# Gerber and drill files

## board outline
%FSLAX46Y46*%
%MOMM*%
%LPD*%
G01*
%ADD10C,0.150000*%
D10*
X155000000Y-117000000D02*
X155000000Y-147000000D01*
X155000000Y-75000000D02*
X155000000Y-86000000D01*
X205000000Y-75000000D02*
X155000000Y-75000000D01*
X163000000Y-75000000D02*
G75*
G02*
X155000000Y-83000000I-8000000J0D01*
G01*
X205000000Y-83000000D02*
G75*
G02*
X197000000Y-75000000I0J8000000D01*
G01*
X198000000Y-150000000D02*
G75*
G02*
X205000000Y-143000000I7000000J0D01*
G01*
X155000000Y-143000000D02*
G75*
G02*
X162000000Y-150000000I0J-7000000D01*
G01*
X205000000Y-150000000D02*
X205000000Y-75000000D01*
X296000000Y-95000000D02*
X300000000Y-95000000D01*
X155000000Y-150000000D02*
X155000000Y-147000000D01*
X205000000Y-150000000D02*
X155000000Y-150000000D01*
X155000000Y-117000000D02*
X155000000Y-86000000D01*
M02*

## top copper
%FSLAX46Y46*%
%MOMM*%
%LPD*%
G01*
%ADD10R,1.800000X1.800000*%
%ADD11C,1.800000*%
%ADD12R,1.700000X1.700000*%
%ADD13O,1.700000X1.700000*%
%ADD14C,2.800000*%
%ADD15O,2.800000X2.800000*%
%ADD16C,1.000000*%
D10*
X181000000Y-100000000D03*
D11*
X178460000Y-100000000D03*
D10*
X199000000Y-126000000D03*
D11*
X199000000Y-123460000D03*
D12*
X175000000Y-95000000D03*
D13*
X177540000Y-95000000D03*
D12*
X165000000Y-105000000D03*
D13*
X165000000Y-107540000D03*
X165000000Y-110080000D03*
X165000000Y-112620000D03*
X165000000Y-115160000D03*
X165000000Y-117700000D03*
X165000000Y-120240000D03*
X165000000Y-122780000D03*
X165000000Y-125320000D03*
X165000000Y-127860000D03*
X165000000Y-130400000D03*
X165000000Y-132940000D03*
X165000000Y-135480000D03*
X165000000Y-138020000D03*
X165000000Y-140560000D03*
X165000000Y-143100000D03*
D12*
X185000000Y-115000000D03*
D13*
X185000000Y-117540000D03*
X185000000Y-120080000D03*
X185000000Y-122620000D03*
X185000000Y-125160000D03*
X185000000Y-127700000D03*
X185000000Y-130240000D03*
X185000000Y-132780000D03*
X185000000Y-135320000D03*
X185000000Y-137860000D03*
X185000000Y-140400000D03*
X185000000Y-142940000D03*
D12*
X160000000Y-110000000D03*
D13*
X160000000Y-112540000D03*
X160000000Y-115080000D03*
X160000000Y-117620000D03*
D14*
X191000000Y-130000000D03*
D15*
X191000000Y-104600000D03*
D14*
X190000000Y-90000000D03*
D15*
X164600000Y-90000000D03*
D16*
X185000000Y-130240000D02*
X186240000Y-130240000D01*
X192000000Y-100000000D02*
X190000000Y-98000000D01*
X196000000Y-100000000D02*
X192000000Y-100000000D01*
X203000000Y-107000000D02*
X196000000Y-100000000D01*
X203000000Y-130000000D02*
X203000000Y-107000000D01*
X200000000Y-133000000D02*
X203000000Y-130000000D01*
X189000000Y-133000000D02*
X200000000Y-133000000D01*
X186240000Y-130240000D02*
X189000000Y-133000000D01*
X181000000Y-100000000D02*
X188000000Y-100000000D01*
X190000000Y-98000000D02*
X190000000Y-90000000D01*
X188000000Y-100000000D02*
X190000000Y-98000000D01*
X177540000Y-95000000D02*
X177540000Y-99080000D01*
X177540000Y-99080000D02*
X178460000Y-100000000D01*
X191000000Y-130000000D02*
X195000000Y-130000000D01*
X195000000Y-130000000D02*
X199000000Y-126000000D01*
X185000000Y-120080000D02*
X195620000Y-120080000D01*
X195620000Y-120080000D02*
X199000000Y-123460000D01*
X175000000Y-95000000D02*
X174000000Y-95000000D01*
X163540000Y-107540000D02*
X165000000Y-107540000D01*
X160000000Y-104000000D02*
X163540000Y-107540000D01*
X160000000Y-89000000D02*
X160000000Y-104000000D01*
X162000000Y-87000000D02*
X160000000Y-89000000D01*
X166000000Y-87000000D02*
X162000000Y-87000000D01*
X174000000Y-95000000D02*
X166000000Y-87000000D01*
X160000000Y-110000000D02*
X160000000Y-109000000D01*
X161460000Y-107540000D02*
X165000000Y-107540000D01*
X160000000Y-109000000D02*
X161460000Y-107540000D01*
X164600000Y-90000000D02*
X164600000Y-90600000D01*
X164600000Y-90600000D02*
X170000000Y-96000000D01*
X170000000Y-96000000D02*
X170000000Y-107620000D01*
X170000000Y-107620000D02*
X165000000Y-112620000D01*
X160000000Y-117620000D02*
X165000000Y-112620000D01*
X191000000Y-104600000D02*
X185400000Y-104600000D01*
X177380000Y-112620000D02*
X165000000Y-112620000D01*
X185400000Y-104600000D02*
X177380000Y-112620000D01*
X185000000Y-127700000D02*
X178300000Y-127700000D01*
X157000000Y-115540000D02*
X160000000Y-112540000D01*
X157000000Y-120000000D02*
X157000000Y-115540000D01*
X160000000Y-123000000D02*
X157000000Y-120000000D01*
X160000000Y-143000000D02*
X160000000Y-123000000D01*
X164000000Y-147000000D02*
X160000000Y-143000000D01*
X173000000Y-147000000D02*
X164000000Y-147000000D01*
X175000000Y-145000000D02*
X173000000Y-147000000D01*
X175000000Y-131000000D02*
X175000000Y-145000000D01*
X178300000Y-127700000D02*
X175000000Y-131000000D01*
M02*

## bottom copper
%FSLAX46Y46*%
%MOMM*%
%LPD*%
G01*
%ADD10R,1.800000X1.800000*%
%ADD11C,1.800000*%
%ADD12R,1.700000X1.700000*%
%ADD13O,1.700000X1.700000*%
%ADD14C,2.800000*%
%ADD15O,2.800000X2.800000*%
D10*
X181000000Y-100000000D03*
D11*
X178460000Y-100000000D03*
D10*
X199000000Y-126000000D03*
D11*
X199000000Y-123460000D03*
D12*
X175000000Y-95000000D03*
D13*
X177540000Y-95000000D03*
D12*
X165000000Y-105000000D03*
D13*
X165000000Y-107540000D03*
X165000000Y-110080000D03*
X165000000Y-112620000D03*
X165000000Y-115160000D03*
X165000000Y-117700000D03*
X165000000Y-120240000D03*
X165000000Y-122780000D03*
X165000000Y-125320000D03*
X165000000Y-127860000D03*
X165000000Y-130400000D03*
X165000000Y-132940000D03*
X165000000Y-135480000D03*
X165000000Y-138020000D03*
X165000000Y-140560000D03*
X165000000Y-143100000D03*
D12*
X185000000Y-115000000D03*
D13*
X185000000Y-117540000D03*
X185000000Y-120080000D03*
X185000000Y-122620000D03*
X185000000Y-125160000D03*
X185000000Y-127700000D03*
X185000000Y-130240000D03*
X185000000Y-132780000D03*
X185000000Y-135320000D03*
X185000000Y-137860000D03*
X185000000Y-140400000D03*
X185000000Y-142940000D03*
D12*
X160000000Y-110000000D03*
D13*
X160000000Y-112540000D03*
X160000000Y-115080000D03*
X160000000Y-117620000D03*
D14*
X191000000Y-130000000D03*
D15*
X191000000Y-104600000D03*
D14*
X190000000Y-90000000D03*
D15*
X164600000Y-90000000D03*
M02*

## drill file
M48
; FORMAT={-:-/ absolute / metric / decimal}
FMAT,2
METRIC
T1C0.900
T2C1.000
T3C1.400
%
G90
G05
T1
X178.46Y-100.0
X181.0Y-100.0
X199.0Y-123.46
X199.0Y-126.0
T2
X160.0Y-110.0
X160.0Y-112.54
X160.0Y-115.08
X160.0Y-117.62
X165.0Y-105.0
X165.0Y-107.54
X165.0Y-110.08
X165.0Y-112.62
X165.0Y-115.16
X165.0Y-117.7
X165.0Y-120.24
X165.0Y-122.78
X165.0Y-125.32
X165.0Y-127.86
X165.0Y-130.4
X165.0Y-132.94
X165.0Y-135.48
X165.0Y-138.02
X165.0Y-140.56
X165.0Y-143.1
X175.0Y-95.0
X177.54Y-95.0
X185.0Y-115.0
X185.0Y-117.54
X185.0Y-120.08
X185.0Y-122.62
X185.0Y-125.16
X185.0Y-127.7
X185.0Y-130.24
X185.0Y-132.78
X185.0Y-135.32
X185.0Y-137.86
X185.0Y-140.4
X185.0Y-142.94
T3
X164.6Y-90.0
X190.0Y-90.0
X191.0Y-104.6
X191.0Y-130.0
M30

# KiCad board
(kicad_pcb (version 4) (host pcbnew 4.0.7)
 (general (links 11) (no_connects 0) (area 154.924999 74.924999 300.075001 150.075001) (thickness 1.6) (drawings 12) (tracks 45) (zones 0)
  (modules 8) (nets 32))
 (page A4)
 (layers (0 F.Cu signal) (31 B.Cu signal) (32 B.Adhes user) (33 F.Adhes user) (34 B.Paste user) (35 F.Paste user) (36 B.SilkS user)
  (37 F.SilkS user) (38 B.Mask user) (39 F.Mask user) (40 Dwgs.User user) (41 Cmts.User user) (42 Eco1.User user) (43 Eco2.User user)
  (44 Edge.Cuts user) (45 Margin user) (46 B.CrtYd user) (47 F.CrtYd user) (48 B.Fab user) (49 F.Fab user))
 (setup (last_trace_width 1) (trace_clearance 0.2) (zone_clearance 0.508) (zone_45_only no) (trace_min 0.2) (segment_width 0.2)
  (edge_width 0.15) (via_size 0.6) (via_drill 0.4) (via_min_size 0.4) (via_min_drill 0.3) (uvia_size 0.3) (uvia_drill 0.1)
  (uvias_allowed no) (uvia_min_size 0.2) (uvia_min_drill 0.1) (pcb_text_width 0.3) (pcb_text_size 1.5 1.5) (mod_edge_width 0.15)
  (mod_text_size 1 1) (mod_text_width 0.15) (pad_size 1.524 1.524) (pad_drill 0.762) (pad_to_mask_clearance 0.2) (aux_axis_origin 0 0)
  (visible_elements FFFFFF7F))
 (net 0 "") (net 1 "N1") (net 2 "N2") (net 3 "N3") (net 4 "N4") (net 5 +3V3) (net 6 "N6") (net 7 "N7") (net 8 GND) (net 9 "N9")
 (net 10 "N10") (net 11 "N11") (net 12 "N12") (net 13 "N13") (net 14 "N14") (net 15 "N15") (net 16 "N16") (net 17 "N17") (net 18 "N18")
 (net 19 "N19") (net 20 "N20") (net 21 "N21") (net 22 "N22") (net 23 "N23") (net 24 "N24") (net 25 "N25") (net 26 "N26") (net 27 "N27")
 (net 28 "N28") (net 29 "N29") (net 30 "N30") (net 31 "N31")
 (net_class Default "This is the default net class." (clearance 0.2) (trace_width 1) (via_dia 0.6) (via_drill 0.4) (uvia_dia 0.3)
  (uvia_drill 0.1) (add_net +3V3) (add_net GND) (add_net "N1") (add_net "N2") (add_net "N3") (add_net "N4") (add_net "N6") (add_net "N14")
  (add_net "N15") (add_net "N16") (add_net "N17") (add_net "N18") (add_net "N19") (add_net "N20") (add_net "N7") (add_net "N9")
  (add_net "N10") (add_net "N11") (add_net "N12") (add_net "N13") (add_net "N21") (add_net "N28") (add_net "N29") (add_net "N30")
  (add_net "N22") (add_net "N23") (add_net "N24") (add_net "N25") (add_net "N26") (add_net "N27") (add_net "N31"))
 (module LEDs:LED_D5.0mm (layer F.Cu) (at 181 100 180)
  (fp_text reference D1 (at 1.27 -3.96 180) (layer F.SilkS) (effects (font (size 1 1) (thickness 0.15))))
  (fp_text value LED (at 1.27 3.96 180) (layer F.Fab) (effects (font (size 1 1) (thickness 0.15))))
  (pad 1 thru_hole rect (at 0 0 180) (size 1.8 1.8) (drill 0.9) (layers *.Cu *.Mask) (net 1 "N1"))
  (pad 2 thru_hole circle (at 2.54 0 180) (size 1.8 1.8) (drill 0.9) (layers *.Cu *.Mask) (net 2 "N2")))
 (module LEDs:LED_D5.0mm (layer F.Cu) (at 199 126 90)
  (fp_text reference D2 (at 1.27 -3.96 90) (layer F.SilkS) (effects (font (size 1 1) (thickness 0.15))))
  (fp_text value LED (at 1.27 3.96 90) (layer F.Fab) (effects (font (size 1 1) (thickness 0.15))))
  (pad 1 thru_hole rect (at 0 0 90) (size 1.8 1.8) (drill 0.9) (layers *.Cu *.Mask) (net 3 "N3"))
  (pad 2 thru_hole circle (at 2.54 0 90) (size 1.8 1.8) (drill 0.9) (layers *.Cu *.Mask) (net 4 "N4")))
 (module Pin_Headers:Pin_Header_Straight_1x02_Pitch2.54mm (layer F.Cu) (at 175 95 90)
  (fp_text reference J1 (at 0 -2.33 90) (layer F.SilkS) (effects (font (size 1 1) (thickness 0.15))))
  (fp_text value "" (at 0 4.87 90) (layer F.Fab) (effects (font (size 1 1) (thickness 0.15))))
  (pad 1 thru_hole rect (at 0 0 90) (size 1.7 1.7) (drill 1) (layers *.Cu *.Mask) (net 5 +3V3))
  (pad 2 thru_hole oval (at 0 2.54 90) (size 1.7 1.7) (drill 1) (layers *.Cu *.Mask) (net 2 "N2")))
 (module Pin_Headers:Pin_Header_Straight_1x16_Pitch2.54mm (layer F.Cu) (at 165 105)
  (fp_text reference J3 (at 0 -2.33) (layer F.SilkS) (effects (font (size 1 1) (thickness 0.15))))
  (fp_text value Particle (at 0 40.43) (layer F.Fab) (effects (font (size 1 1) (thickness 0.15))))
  (pad 1 thru_hole rect (at 0 0) (size 1.7 1.7) (drill 1) (layers *.Cu *.Mask) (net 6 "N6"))
  (pad 2 thru_hole oval (at 0 2.54) (size 1.7 1.7) (drill 1) (layers *.Cu *.Mask) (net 5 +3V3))
  (pad 3 thru_hole oval (at 0 5.08) (size 1.7 1.7) (drill 1) (layers *.Cu *.Mask) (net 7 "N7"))
  (pad 4 thru_hole oval (at 0 7.62) (size 1.7 1.7) (drill 1) (layers *.Cu *.Mask) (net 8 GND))
  (pad 5 thru_hole oval (at 0 10.16) (size 1.7 1.7) (drill 1) (layers *.Cu *.Mask) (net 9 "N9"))
  (pad 6 thru_hole oval (at 0 12.7) (size 1.7 1.7) (drill 1) (layers *.Cu *.Mask) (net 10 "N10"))
  (pad 7 thru_hole oval (at 0 15.24) (size 1.7 1.7) (drill 1) (layers *.Cu *.Mask) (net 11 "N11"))
  (pad 8 thru_hole oval (at 0 17.78) (size 1.7 1.7) (drill 1) (layers *.Cu *.Mask) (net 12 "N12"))
  (pad 9 thru_hole oval (at 0 20.32) (size 1.7 1.7) (drill 1) (layers *.Cu *.Mask) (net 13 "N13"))
  (pad 10 thru_hole oval (at 0 22.86) (size 1.7 1.7) (drill 1) (layers *.Cu *.Mask) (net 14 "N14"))
  (pad 11 thru_hole oval (at 0 25.4) (size 1.7 1.7) (drill 1) (layers *.Cu *.Mask) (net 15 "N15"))
  (pad 12 thru_hole oval (at 0 27.94) (size 1.7 1.7) (drill 1) (layers *.Cu *.Mask) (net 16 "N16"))
  (pad 13 thru_hole oval (at 0 30.48) (size 1.7 1.7) (drill 1) (layers *.Cu *.Mask) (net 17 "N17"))
  (pad 14 thru_hole oval (at 0 33.02) (size 1.7 1.7) (drill 1) (layers *.Cu *.Mask) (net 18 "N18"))
  (pad 15 thru_hole oval (at 0 35.56) (size 1.7 1.7) (drill 1) (layers *.Cu *.Mask) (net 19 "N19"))
  (pad 16 thru_hole oval (at 0 38.1) (size 1.7 1.7) (drill 1) (layers *.Cu *.Mask) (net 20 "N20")))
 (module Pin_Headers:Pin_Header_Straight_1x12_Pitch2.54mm (layer F.Cu) (at 185 115)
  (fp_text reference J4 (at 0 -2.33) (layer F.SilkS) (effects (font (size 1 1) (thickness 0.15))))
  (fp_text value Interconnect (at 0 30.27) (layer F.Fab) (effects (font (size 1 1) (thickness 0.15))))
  (pad 1 thru_hole rect (at 0 0) (size 1.7 1.7) (drill 1) (layers *.Cu *.Mask) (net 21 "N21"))
  (pad 2 thru_hole oval (at 0 2.54) (size 1.7 1.7) (drill 1) (layers *.Cu *.Mask) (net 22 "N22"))
  (pad 3 thru_hole oval (at 0 5.08) (size 1.7 1.7) (drill 1) (layers *.Cu *.Mask) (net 4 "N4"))
  (pad 4 thru_hole oval (at 0 7.62) (size 1.7 1.7) (drill 1) (layers *.Cu *.Mask) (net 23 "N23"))
  (pad 5 thru_hole oval (at 0 10.16) (size 1.7 1.7) (drill 1) (layers *.Cu *.Mask) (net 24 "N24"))
  (pad 6 thru_hole oval (at 0 12.7) (size 1.7 1.7) (drill 1) (layers *.Cu *.Mask) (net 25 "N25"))
  (pad 7 thru_hole oval (at 0 15.24) (size 1.7 1.7) (drill 1) (layers *.Cu *.Mask) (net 1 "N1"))
  (pad 8 thru_hole oval (at 0 17.78) (size 1.7 1.7) (drill 1) (layers *.Cu *.Mask) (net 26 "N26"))
  (pad 9 thru_hole oval (at 0 20.32) (size 1.7 1.7) (drill 1) (layers *.Cu *.Mask) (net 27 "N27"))
  (pad 10 thru_hole oval (at 0 22.86) (size 1.7 1.7) (drill 1) (layers *.Cu *.Mask) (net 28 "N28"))
  (pad 11 thru_hole oval (at 0 25.4) (size 1.7 1.7) (drill 1) (layers *.Cu *.Mask) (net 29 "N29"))
  (pad 12 thru_hole oval (at 0 27.94) (size 1.7 1.7) (drill 1) (layers *.Cu *.Mask) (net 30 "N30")))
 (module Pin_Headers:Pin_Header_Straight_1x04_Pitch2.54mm (layer F.Cu) (at 160 110)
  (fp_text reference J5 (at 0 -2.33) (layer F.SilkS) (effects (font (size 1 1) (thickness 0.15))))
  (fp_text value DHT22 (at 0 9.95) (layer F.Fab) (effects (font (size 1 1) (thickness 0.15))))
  (pad 1 thru_hole rect (at 0 0) (size 1.7 1.7) (drill 1) (layers *.Cu *.Mask) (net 5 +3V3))
  (pad 2 thru_hole oval (at 0 2.54) (size 1.7 1.7) (drill 1) (layers *.Cu *.Mask) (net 25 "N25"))
  (pad 3 thru_hole oval (at 0 5.08) (size 1.7 1.7) (drill 1) (layers *.Cu *.Mask) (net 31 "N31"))
  (pad 4 thru_hole oval (at 0 7.62) (size 1.7 1.7) (drill 1) (layers *.Cu *.Mask) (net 8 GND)))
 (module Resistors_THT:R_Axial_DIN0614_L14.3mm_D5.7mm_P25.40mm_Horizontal (layer F.Cu) (at 191 130 90)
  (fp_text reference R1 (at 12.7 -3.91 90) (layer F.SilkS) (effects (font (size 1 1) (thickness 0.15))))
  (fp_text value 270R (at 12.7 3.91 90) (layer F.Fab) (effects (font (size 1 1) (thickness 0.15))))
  (pad 1 thru_hole circle (at 0 0 90) (size 2.8 2.8) (drill 1.4) (layers *.Cu *.Mask) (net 3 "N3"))
  (pad 2 thru_hole oval (at 25.4 0 90) (size 2.8 2.8) (drill 1.4) (layers *.Cu *.Mask) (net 8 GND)))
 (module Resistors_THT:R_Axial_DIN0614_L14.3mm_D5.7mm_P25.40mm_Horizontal (layer F.Cu) (at 190 90 180)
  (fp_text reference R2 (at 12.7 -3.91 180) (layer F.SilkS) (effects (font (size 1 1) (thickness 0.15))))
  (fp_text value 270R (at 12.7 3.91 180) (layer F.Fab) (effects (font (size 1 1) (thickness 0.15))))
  (pad 1 thru_hole circle (at 0 0 180) (size 2.8 2.8) (drill 1.4) (layers *.Cu *.Mask) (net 1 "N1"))
  (pad 2 thru_hole oval (at 25.4 0 180) (size 2.8 2.8) (drill 1.4) (layers *.Cu *.Mask) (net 8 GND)))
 (gr_line (start 155 117) (end 155 147) (angle 90) (layer Edge.Cuts) (width 0.15))
 (gr_line (start 155 75) (end 155 86) (angle 90) (layer Edge.Cuts) (width 0.15))
 (gr_line (start 205 75) (end 155 75) (angle 90) (layer Edge.Cuts) (width 0.15))
 (gr_arc (start 155 75) (end 163 75) (angle 90) (layer Edge.Cuts) (width 0.15))
 (gr_arc (start 205 75) (end 205 83) (angle 90) (layer Edge.Cuts) (width 0.15))
 (gr_arc (start 205 150) (end 198 150) (angle 90) (layer Edge.Cuts) (width 0.15))
 (gr_arc (start 155 150) (end 155 143) (angle 90) (layer Edge.Cuts) (width 0.15))
 (gr_line (start 205 150) (end 205 75) (angle 90) (layer Edge.Cuts) (width 0.15))
 (gr_line (start 296 95) (end 300 95) (angle 90) (layer Edge.Cuts) (width 0.15))
 (gr_line (start 155 150) (end 155 147) (angle 90) (layer Edge.Cuts) (width 0.15))
 (gr_line (start 205 150) (end 155 150) (angle 90) (layer Edge.Cuts) (width 0.15))
 (gr_line (start 155 117) (end 155 86) (angle 90) (layer Edge.Cuts) (width 0.15))
 (segment (start 185 130.24) (end 186.24 130.24) (width 1) (layer F.Cu) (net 1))
 (segment (start 192 100) (end 190 98) (width 1) (layer F.Cu) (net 1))
 (segment (start 196 100) (end 192 100) (width 1) (layer F.Cu) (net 1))
 (segment (start 203 107) (end 196 100) (width 1) (layer F.Cu) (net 1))
 (segment (start 203 130) (end 203 107) (width 1) (layer F.Cu) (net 1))
 (segment (start 200 133) (end 203 130) (width 1) (layer F.Cu) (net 1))
 (segment (start 189 133) (end 200 133) (width 1) (layer F.Cu) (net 1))
 (segment (start 186.24 130.24) (end 189 133) (width 1) (layer F.Cu) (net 1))
 (segment (start 181 100) (end 188 100) (width 1) (layer F.Cu) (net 1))
 (segment (start 190 98) (end 190 90) (width 1) (layer F.Cu) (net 1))
 (segment (start 188 100) (end 190 98) (width 1) (layer F.Cu) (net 1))
 (segment (start 177.54 95) (end 177.54 99.08) (width 1) (layer F.Cu) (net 2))
 (segment (start 177.54 99.08) (end 178.46 100) (width 1) (layer F.Cu) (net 2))
 (segment (start 191 130) (end 195 130) (width 1) (layer F.Cu) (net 3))
 (segment (start 195 130) (end 199 126) (width 1) (layer F.Cu) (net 3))
 (segment (start 185 120.08) (end 195.62 120.08) (width 1) (layer F.Cu) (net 4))
 (segment (start 195.62 120.08) (end 199 123.46) (width 1) (layer F.Cu) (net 4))
 (segment (start 175 95) (end 174 95) (width 1) (layer F.Cu) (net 5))
 (segment (start 163.54 107.54) (end 165 107.54) (width 1) (layer F.Cu) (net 5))
 (segment (start 160 104) (end 163.54 107.54) (width 1) (layer F.Cu) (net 5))
 (segment (start 160 89) (end 160 104) (width 1) (layer F.Cu) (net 5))
 (segment (start 162 87) (end 160 89) (width 1) (layer F.Cu) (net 5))
 (segment (start 166 87) (end 162 87) (width 1) (layer F.Cu) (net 5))
 (segment (start 174 95) (end 166 87) (width 1) (layer F.Cu) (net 5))
 (segment (start 160 110) (end 160 109) (width 1) (layer F.Cu) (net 5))
 (segment (start 161.46 107.54) (end 165 107.54) (width 1) (layer F.Cu) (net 5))
 (segment (start 160 109) (end 161.46 107.54) (width 1) (layer F.Cu) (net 5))
 (segment (start 164.6 90) (end 164.6 90.6) (width 1) (layer F.Cu) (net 8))
 (segment (start 164.6 90.6) (end 170 96) (width 1) (layer F.Cu) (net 8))
 (segment (start 170 96) (end 170 107.62) (width 1) (layer F.Cu) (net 8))
 (segment (start 170 107.62) (end 165 112.62) (width 1) (layer F.Cu) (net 8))
 (segment (start 160 117.62) (end 165 112.62) (width 1) (layer F.Cu) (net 8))
 (segment (start 191 104.6) (end 185.4 104.6) (width 1) (layer F.Cu) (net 8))
 (segment (start 177.38 112.62) (end 165 112.62) (width 1) (layer F.Cu) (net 8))
 (segment (start 185.4 104.6) (end 177.38 112.62) (width 1) (layer F.Cu) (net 8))
 (segment (start 185 127.7) (end 178.3 127.7) (width 1) (layer F.Cu) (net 25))
 (segment (start 157 115.54) (end 160 112.54) (width 1) (layer F.Cu) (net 25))
 (segment (start 157 120) (end 157 115.54) (width 1) (layer F.Cu) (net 25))
 (segment (start 160 123) (end 157 120) (width 1) (layer F.Cu) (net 25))
 (segment (start 160 143) (end 160 123) (width 1) (layer F.Cu) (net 25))
 (segment (start 164 147) (end 160 143) (width 1) (layer F.Cu) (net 25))
 (segment (start 173 147) (end 164 147) (width 1) (layer F.Cu) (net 25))
 (segment (start 175 145) (end 173 147) (width 1) (layer F.Cu) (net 25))
 (segment (start 175 131) (end 175 145) (width 1) (layer F.Cu) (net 25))
 (segment (start 178.3 127.7) (end 175 131) (width 1) (layer F.Cu) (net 25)))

